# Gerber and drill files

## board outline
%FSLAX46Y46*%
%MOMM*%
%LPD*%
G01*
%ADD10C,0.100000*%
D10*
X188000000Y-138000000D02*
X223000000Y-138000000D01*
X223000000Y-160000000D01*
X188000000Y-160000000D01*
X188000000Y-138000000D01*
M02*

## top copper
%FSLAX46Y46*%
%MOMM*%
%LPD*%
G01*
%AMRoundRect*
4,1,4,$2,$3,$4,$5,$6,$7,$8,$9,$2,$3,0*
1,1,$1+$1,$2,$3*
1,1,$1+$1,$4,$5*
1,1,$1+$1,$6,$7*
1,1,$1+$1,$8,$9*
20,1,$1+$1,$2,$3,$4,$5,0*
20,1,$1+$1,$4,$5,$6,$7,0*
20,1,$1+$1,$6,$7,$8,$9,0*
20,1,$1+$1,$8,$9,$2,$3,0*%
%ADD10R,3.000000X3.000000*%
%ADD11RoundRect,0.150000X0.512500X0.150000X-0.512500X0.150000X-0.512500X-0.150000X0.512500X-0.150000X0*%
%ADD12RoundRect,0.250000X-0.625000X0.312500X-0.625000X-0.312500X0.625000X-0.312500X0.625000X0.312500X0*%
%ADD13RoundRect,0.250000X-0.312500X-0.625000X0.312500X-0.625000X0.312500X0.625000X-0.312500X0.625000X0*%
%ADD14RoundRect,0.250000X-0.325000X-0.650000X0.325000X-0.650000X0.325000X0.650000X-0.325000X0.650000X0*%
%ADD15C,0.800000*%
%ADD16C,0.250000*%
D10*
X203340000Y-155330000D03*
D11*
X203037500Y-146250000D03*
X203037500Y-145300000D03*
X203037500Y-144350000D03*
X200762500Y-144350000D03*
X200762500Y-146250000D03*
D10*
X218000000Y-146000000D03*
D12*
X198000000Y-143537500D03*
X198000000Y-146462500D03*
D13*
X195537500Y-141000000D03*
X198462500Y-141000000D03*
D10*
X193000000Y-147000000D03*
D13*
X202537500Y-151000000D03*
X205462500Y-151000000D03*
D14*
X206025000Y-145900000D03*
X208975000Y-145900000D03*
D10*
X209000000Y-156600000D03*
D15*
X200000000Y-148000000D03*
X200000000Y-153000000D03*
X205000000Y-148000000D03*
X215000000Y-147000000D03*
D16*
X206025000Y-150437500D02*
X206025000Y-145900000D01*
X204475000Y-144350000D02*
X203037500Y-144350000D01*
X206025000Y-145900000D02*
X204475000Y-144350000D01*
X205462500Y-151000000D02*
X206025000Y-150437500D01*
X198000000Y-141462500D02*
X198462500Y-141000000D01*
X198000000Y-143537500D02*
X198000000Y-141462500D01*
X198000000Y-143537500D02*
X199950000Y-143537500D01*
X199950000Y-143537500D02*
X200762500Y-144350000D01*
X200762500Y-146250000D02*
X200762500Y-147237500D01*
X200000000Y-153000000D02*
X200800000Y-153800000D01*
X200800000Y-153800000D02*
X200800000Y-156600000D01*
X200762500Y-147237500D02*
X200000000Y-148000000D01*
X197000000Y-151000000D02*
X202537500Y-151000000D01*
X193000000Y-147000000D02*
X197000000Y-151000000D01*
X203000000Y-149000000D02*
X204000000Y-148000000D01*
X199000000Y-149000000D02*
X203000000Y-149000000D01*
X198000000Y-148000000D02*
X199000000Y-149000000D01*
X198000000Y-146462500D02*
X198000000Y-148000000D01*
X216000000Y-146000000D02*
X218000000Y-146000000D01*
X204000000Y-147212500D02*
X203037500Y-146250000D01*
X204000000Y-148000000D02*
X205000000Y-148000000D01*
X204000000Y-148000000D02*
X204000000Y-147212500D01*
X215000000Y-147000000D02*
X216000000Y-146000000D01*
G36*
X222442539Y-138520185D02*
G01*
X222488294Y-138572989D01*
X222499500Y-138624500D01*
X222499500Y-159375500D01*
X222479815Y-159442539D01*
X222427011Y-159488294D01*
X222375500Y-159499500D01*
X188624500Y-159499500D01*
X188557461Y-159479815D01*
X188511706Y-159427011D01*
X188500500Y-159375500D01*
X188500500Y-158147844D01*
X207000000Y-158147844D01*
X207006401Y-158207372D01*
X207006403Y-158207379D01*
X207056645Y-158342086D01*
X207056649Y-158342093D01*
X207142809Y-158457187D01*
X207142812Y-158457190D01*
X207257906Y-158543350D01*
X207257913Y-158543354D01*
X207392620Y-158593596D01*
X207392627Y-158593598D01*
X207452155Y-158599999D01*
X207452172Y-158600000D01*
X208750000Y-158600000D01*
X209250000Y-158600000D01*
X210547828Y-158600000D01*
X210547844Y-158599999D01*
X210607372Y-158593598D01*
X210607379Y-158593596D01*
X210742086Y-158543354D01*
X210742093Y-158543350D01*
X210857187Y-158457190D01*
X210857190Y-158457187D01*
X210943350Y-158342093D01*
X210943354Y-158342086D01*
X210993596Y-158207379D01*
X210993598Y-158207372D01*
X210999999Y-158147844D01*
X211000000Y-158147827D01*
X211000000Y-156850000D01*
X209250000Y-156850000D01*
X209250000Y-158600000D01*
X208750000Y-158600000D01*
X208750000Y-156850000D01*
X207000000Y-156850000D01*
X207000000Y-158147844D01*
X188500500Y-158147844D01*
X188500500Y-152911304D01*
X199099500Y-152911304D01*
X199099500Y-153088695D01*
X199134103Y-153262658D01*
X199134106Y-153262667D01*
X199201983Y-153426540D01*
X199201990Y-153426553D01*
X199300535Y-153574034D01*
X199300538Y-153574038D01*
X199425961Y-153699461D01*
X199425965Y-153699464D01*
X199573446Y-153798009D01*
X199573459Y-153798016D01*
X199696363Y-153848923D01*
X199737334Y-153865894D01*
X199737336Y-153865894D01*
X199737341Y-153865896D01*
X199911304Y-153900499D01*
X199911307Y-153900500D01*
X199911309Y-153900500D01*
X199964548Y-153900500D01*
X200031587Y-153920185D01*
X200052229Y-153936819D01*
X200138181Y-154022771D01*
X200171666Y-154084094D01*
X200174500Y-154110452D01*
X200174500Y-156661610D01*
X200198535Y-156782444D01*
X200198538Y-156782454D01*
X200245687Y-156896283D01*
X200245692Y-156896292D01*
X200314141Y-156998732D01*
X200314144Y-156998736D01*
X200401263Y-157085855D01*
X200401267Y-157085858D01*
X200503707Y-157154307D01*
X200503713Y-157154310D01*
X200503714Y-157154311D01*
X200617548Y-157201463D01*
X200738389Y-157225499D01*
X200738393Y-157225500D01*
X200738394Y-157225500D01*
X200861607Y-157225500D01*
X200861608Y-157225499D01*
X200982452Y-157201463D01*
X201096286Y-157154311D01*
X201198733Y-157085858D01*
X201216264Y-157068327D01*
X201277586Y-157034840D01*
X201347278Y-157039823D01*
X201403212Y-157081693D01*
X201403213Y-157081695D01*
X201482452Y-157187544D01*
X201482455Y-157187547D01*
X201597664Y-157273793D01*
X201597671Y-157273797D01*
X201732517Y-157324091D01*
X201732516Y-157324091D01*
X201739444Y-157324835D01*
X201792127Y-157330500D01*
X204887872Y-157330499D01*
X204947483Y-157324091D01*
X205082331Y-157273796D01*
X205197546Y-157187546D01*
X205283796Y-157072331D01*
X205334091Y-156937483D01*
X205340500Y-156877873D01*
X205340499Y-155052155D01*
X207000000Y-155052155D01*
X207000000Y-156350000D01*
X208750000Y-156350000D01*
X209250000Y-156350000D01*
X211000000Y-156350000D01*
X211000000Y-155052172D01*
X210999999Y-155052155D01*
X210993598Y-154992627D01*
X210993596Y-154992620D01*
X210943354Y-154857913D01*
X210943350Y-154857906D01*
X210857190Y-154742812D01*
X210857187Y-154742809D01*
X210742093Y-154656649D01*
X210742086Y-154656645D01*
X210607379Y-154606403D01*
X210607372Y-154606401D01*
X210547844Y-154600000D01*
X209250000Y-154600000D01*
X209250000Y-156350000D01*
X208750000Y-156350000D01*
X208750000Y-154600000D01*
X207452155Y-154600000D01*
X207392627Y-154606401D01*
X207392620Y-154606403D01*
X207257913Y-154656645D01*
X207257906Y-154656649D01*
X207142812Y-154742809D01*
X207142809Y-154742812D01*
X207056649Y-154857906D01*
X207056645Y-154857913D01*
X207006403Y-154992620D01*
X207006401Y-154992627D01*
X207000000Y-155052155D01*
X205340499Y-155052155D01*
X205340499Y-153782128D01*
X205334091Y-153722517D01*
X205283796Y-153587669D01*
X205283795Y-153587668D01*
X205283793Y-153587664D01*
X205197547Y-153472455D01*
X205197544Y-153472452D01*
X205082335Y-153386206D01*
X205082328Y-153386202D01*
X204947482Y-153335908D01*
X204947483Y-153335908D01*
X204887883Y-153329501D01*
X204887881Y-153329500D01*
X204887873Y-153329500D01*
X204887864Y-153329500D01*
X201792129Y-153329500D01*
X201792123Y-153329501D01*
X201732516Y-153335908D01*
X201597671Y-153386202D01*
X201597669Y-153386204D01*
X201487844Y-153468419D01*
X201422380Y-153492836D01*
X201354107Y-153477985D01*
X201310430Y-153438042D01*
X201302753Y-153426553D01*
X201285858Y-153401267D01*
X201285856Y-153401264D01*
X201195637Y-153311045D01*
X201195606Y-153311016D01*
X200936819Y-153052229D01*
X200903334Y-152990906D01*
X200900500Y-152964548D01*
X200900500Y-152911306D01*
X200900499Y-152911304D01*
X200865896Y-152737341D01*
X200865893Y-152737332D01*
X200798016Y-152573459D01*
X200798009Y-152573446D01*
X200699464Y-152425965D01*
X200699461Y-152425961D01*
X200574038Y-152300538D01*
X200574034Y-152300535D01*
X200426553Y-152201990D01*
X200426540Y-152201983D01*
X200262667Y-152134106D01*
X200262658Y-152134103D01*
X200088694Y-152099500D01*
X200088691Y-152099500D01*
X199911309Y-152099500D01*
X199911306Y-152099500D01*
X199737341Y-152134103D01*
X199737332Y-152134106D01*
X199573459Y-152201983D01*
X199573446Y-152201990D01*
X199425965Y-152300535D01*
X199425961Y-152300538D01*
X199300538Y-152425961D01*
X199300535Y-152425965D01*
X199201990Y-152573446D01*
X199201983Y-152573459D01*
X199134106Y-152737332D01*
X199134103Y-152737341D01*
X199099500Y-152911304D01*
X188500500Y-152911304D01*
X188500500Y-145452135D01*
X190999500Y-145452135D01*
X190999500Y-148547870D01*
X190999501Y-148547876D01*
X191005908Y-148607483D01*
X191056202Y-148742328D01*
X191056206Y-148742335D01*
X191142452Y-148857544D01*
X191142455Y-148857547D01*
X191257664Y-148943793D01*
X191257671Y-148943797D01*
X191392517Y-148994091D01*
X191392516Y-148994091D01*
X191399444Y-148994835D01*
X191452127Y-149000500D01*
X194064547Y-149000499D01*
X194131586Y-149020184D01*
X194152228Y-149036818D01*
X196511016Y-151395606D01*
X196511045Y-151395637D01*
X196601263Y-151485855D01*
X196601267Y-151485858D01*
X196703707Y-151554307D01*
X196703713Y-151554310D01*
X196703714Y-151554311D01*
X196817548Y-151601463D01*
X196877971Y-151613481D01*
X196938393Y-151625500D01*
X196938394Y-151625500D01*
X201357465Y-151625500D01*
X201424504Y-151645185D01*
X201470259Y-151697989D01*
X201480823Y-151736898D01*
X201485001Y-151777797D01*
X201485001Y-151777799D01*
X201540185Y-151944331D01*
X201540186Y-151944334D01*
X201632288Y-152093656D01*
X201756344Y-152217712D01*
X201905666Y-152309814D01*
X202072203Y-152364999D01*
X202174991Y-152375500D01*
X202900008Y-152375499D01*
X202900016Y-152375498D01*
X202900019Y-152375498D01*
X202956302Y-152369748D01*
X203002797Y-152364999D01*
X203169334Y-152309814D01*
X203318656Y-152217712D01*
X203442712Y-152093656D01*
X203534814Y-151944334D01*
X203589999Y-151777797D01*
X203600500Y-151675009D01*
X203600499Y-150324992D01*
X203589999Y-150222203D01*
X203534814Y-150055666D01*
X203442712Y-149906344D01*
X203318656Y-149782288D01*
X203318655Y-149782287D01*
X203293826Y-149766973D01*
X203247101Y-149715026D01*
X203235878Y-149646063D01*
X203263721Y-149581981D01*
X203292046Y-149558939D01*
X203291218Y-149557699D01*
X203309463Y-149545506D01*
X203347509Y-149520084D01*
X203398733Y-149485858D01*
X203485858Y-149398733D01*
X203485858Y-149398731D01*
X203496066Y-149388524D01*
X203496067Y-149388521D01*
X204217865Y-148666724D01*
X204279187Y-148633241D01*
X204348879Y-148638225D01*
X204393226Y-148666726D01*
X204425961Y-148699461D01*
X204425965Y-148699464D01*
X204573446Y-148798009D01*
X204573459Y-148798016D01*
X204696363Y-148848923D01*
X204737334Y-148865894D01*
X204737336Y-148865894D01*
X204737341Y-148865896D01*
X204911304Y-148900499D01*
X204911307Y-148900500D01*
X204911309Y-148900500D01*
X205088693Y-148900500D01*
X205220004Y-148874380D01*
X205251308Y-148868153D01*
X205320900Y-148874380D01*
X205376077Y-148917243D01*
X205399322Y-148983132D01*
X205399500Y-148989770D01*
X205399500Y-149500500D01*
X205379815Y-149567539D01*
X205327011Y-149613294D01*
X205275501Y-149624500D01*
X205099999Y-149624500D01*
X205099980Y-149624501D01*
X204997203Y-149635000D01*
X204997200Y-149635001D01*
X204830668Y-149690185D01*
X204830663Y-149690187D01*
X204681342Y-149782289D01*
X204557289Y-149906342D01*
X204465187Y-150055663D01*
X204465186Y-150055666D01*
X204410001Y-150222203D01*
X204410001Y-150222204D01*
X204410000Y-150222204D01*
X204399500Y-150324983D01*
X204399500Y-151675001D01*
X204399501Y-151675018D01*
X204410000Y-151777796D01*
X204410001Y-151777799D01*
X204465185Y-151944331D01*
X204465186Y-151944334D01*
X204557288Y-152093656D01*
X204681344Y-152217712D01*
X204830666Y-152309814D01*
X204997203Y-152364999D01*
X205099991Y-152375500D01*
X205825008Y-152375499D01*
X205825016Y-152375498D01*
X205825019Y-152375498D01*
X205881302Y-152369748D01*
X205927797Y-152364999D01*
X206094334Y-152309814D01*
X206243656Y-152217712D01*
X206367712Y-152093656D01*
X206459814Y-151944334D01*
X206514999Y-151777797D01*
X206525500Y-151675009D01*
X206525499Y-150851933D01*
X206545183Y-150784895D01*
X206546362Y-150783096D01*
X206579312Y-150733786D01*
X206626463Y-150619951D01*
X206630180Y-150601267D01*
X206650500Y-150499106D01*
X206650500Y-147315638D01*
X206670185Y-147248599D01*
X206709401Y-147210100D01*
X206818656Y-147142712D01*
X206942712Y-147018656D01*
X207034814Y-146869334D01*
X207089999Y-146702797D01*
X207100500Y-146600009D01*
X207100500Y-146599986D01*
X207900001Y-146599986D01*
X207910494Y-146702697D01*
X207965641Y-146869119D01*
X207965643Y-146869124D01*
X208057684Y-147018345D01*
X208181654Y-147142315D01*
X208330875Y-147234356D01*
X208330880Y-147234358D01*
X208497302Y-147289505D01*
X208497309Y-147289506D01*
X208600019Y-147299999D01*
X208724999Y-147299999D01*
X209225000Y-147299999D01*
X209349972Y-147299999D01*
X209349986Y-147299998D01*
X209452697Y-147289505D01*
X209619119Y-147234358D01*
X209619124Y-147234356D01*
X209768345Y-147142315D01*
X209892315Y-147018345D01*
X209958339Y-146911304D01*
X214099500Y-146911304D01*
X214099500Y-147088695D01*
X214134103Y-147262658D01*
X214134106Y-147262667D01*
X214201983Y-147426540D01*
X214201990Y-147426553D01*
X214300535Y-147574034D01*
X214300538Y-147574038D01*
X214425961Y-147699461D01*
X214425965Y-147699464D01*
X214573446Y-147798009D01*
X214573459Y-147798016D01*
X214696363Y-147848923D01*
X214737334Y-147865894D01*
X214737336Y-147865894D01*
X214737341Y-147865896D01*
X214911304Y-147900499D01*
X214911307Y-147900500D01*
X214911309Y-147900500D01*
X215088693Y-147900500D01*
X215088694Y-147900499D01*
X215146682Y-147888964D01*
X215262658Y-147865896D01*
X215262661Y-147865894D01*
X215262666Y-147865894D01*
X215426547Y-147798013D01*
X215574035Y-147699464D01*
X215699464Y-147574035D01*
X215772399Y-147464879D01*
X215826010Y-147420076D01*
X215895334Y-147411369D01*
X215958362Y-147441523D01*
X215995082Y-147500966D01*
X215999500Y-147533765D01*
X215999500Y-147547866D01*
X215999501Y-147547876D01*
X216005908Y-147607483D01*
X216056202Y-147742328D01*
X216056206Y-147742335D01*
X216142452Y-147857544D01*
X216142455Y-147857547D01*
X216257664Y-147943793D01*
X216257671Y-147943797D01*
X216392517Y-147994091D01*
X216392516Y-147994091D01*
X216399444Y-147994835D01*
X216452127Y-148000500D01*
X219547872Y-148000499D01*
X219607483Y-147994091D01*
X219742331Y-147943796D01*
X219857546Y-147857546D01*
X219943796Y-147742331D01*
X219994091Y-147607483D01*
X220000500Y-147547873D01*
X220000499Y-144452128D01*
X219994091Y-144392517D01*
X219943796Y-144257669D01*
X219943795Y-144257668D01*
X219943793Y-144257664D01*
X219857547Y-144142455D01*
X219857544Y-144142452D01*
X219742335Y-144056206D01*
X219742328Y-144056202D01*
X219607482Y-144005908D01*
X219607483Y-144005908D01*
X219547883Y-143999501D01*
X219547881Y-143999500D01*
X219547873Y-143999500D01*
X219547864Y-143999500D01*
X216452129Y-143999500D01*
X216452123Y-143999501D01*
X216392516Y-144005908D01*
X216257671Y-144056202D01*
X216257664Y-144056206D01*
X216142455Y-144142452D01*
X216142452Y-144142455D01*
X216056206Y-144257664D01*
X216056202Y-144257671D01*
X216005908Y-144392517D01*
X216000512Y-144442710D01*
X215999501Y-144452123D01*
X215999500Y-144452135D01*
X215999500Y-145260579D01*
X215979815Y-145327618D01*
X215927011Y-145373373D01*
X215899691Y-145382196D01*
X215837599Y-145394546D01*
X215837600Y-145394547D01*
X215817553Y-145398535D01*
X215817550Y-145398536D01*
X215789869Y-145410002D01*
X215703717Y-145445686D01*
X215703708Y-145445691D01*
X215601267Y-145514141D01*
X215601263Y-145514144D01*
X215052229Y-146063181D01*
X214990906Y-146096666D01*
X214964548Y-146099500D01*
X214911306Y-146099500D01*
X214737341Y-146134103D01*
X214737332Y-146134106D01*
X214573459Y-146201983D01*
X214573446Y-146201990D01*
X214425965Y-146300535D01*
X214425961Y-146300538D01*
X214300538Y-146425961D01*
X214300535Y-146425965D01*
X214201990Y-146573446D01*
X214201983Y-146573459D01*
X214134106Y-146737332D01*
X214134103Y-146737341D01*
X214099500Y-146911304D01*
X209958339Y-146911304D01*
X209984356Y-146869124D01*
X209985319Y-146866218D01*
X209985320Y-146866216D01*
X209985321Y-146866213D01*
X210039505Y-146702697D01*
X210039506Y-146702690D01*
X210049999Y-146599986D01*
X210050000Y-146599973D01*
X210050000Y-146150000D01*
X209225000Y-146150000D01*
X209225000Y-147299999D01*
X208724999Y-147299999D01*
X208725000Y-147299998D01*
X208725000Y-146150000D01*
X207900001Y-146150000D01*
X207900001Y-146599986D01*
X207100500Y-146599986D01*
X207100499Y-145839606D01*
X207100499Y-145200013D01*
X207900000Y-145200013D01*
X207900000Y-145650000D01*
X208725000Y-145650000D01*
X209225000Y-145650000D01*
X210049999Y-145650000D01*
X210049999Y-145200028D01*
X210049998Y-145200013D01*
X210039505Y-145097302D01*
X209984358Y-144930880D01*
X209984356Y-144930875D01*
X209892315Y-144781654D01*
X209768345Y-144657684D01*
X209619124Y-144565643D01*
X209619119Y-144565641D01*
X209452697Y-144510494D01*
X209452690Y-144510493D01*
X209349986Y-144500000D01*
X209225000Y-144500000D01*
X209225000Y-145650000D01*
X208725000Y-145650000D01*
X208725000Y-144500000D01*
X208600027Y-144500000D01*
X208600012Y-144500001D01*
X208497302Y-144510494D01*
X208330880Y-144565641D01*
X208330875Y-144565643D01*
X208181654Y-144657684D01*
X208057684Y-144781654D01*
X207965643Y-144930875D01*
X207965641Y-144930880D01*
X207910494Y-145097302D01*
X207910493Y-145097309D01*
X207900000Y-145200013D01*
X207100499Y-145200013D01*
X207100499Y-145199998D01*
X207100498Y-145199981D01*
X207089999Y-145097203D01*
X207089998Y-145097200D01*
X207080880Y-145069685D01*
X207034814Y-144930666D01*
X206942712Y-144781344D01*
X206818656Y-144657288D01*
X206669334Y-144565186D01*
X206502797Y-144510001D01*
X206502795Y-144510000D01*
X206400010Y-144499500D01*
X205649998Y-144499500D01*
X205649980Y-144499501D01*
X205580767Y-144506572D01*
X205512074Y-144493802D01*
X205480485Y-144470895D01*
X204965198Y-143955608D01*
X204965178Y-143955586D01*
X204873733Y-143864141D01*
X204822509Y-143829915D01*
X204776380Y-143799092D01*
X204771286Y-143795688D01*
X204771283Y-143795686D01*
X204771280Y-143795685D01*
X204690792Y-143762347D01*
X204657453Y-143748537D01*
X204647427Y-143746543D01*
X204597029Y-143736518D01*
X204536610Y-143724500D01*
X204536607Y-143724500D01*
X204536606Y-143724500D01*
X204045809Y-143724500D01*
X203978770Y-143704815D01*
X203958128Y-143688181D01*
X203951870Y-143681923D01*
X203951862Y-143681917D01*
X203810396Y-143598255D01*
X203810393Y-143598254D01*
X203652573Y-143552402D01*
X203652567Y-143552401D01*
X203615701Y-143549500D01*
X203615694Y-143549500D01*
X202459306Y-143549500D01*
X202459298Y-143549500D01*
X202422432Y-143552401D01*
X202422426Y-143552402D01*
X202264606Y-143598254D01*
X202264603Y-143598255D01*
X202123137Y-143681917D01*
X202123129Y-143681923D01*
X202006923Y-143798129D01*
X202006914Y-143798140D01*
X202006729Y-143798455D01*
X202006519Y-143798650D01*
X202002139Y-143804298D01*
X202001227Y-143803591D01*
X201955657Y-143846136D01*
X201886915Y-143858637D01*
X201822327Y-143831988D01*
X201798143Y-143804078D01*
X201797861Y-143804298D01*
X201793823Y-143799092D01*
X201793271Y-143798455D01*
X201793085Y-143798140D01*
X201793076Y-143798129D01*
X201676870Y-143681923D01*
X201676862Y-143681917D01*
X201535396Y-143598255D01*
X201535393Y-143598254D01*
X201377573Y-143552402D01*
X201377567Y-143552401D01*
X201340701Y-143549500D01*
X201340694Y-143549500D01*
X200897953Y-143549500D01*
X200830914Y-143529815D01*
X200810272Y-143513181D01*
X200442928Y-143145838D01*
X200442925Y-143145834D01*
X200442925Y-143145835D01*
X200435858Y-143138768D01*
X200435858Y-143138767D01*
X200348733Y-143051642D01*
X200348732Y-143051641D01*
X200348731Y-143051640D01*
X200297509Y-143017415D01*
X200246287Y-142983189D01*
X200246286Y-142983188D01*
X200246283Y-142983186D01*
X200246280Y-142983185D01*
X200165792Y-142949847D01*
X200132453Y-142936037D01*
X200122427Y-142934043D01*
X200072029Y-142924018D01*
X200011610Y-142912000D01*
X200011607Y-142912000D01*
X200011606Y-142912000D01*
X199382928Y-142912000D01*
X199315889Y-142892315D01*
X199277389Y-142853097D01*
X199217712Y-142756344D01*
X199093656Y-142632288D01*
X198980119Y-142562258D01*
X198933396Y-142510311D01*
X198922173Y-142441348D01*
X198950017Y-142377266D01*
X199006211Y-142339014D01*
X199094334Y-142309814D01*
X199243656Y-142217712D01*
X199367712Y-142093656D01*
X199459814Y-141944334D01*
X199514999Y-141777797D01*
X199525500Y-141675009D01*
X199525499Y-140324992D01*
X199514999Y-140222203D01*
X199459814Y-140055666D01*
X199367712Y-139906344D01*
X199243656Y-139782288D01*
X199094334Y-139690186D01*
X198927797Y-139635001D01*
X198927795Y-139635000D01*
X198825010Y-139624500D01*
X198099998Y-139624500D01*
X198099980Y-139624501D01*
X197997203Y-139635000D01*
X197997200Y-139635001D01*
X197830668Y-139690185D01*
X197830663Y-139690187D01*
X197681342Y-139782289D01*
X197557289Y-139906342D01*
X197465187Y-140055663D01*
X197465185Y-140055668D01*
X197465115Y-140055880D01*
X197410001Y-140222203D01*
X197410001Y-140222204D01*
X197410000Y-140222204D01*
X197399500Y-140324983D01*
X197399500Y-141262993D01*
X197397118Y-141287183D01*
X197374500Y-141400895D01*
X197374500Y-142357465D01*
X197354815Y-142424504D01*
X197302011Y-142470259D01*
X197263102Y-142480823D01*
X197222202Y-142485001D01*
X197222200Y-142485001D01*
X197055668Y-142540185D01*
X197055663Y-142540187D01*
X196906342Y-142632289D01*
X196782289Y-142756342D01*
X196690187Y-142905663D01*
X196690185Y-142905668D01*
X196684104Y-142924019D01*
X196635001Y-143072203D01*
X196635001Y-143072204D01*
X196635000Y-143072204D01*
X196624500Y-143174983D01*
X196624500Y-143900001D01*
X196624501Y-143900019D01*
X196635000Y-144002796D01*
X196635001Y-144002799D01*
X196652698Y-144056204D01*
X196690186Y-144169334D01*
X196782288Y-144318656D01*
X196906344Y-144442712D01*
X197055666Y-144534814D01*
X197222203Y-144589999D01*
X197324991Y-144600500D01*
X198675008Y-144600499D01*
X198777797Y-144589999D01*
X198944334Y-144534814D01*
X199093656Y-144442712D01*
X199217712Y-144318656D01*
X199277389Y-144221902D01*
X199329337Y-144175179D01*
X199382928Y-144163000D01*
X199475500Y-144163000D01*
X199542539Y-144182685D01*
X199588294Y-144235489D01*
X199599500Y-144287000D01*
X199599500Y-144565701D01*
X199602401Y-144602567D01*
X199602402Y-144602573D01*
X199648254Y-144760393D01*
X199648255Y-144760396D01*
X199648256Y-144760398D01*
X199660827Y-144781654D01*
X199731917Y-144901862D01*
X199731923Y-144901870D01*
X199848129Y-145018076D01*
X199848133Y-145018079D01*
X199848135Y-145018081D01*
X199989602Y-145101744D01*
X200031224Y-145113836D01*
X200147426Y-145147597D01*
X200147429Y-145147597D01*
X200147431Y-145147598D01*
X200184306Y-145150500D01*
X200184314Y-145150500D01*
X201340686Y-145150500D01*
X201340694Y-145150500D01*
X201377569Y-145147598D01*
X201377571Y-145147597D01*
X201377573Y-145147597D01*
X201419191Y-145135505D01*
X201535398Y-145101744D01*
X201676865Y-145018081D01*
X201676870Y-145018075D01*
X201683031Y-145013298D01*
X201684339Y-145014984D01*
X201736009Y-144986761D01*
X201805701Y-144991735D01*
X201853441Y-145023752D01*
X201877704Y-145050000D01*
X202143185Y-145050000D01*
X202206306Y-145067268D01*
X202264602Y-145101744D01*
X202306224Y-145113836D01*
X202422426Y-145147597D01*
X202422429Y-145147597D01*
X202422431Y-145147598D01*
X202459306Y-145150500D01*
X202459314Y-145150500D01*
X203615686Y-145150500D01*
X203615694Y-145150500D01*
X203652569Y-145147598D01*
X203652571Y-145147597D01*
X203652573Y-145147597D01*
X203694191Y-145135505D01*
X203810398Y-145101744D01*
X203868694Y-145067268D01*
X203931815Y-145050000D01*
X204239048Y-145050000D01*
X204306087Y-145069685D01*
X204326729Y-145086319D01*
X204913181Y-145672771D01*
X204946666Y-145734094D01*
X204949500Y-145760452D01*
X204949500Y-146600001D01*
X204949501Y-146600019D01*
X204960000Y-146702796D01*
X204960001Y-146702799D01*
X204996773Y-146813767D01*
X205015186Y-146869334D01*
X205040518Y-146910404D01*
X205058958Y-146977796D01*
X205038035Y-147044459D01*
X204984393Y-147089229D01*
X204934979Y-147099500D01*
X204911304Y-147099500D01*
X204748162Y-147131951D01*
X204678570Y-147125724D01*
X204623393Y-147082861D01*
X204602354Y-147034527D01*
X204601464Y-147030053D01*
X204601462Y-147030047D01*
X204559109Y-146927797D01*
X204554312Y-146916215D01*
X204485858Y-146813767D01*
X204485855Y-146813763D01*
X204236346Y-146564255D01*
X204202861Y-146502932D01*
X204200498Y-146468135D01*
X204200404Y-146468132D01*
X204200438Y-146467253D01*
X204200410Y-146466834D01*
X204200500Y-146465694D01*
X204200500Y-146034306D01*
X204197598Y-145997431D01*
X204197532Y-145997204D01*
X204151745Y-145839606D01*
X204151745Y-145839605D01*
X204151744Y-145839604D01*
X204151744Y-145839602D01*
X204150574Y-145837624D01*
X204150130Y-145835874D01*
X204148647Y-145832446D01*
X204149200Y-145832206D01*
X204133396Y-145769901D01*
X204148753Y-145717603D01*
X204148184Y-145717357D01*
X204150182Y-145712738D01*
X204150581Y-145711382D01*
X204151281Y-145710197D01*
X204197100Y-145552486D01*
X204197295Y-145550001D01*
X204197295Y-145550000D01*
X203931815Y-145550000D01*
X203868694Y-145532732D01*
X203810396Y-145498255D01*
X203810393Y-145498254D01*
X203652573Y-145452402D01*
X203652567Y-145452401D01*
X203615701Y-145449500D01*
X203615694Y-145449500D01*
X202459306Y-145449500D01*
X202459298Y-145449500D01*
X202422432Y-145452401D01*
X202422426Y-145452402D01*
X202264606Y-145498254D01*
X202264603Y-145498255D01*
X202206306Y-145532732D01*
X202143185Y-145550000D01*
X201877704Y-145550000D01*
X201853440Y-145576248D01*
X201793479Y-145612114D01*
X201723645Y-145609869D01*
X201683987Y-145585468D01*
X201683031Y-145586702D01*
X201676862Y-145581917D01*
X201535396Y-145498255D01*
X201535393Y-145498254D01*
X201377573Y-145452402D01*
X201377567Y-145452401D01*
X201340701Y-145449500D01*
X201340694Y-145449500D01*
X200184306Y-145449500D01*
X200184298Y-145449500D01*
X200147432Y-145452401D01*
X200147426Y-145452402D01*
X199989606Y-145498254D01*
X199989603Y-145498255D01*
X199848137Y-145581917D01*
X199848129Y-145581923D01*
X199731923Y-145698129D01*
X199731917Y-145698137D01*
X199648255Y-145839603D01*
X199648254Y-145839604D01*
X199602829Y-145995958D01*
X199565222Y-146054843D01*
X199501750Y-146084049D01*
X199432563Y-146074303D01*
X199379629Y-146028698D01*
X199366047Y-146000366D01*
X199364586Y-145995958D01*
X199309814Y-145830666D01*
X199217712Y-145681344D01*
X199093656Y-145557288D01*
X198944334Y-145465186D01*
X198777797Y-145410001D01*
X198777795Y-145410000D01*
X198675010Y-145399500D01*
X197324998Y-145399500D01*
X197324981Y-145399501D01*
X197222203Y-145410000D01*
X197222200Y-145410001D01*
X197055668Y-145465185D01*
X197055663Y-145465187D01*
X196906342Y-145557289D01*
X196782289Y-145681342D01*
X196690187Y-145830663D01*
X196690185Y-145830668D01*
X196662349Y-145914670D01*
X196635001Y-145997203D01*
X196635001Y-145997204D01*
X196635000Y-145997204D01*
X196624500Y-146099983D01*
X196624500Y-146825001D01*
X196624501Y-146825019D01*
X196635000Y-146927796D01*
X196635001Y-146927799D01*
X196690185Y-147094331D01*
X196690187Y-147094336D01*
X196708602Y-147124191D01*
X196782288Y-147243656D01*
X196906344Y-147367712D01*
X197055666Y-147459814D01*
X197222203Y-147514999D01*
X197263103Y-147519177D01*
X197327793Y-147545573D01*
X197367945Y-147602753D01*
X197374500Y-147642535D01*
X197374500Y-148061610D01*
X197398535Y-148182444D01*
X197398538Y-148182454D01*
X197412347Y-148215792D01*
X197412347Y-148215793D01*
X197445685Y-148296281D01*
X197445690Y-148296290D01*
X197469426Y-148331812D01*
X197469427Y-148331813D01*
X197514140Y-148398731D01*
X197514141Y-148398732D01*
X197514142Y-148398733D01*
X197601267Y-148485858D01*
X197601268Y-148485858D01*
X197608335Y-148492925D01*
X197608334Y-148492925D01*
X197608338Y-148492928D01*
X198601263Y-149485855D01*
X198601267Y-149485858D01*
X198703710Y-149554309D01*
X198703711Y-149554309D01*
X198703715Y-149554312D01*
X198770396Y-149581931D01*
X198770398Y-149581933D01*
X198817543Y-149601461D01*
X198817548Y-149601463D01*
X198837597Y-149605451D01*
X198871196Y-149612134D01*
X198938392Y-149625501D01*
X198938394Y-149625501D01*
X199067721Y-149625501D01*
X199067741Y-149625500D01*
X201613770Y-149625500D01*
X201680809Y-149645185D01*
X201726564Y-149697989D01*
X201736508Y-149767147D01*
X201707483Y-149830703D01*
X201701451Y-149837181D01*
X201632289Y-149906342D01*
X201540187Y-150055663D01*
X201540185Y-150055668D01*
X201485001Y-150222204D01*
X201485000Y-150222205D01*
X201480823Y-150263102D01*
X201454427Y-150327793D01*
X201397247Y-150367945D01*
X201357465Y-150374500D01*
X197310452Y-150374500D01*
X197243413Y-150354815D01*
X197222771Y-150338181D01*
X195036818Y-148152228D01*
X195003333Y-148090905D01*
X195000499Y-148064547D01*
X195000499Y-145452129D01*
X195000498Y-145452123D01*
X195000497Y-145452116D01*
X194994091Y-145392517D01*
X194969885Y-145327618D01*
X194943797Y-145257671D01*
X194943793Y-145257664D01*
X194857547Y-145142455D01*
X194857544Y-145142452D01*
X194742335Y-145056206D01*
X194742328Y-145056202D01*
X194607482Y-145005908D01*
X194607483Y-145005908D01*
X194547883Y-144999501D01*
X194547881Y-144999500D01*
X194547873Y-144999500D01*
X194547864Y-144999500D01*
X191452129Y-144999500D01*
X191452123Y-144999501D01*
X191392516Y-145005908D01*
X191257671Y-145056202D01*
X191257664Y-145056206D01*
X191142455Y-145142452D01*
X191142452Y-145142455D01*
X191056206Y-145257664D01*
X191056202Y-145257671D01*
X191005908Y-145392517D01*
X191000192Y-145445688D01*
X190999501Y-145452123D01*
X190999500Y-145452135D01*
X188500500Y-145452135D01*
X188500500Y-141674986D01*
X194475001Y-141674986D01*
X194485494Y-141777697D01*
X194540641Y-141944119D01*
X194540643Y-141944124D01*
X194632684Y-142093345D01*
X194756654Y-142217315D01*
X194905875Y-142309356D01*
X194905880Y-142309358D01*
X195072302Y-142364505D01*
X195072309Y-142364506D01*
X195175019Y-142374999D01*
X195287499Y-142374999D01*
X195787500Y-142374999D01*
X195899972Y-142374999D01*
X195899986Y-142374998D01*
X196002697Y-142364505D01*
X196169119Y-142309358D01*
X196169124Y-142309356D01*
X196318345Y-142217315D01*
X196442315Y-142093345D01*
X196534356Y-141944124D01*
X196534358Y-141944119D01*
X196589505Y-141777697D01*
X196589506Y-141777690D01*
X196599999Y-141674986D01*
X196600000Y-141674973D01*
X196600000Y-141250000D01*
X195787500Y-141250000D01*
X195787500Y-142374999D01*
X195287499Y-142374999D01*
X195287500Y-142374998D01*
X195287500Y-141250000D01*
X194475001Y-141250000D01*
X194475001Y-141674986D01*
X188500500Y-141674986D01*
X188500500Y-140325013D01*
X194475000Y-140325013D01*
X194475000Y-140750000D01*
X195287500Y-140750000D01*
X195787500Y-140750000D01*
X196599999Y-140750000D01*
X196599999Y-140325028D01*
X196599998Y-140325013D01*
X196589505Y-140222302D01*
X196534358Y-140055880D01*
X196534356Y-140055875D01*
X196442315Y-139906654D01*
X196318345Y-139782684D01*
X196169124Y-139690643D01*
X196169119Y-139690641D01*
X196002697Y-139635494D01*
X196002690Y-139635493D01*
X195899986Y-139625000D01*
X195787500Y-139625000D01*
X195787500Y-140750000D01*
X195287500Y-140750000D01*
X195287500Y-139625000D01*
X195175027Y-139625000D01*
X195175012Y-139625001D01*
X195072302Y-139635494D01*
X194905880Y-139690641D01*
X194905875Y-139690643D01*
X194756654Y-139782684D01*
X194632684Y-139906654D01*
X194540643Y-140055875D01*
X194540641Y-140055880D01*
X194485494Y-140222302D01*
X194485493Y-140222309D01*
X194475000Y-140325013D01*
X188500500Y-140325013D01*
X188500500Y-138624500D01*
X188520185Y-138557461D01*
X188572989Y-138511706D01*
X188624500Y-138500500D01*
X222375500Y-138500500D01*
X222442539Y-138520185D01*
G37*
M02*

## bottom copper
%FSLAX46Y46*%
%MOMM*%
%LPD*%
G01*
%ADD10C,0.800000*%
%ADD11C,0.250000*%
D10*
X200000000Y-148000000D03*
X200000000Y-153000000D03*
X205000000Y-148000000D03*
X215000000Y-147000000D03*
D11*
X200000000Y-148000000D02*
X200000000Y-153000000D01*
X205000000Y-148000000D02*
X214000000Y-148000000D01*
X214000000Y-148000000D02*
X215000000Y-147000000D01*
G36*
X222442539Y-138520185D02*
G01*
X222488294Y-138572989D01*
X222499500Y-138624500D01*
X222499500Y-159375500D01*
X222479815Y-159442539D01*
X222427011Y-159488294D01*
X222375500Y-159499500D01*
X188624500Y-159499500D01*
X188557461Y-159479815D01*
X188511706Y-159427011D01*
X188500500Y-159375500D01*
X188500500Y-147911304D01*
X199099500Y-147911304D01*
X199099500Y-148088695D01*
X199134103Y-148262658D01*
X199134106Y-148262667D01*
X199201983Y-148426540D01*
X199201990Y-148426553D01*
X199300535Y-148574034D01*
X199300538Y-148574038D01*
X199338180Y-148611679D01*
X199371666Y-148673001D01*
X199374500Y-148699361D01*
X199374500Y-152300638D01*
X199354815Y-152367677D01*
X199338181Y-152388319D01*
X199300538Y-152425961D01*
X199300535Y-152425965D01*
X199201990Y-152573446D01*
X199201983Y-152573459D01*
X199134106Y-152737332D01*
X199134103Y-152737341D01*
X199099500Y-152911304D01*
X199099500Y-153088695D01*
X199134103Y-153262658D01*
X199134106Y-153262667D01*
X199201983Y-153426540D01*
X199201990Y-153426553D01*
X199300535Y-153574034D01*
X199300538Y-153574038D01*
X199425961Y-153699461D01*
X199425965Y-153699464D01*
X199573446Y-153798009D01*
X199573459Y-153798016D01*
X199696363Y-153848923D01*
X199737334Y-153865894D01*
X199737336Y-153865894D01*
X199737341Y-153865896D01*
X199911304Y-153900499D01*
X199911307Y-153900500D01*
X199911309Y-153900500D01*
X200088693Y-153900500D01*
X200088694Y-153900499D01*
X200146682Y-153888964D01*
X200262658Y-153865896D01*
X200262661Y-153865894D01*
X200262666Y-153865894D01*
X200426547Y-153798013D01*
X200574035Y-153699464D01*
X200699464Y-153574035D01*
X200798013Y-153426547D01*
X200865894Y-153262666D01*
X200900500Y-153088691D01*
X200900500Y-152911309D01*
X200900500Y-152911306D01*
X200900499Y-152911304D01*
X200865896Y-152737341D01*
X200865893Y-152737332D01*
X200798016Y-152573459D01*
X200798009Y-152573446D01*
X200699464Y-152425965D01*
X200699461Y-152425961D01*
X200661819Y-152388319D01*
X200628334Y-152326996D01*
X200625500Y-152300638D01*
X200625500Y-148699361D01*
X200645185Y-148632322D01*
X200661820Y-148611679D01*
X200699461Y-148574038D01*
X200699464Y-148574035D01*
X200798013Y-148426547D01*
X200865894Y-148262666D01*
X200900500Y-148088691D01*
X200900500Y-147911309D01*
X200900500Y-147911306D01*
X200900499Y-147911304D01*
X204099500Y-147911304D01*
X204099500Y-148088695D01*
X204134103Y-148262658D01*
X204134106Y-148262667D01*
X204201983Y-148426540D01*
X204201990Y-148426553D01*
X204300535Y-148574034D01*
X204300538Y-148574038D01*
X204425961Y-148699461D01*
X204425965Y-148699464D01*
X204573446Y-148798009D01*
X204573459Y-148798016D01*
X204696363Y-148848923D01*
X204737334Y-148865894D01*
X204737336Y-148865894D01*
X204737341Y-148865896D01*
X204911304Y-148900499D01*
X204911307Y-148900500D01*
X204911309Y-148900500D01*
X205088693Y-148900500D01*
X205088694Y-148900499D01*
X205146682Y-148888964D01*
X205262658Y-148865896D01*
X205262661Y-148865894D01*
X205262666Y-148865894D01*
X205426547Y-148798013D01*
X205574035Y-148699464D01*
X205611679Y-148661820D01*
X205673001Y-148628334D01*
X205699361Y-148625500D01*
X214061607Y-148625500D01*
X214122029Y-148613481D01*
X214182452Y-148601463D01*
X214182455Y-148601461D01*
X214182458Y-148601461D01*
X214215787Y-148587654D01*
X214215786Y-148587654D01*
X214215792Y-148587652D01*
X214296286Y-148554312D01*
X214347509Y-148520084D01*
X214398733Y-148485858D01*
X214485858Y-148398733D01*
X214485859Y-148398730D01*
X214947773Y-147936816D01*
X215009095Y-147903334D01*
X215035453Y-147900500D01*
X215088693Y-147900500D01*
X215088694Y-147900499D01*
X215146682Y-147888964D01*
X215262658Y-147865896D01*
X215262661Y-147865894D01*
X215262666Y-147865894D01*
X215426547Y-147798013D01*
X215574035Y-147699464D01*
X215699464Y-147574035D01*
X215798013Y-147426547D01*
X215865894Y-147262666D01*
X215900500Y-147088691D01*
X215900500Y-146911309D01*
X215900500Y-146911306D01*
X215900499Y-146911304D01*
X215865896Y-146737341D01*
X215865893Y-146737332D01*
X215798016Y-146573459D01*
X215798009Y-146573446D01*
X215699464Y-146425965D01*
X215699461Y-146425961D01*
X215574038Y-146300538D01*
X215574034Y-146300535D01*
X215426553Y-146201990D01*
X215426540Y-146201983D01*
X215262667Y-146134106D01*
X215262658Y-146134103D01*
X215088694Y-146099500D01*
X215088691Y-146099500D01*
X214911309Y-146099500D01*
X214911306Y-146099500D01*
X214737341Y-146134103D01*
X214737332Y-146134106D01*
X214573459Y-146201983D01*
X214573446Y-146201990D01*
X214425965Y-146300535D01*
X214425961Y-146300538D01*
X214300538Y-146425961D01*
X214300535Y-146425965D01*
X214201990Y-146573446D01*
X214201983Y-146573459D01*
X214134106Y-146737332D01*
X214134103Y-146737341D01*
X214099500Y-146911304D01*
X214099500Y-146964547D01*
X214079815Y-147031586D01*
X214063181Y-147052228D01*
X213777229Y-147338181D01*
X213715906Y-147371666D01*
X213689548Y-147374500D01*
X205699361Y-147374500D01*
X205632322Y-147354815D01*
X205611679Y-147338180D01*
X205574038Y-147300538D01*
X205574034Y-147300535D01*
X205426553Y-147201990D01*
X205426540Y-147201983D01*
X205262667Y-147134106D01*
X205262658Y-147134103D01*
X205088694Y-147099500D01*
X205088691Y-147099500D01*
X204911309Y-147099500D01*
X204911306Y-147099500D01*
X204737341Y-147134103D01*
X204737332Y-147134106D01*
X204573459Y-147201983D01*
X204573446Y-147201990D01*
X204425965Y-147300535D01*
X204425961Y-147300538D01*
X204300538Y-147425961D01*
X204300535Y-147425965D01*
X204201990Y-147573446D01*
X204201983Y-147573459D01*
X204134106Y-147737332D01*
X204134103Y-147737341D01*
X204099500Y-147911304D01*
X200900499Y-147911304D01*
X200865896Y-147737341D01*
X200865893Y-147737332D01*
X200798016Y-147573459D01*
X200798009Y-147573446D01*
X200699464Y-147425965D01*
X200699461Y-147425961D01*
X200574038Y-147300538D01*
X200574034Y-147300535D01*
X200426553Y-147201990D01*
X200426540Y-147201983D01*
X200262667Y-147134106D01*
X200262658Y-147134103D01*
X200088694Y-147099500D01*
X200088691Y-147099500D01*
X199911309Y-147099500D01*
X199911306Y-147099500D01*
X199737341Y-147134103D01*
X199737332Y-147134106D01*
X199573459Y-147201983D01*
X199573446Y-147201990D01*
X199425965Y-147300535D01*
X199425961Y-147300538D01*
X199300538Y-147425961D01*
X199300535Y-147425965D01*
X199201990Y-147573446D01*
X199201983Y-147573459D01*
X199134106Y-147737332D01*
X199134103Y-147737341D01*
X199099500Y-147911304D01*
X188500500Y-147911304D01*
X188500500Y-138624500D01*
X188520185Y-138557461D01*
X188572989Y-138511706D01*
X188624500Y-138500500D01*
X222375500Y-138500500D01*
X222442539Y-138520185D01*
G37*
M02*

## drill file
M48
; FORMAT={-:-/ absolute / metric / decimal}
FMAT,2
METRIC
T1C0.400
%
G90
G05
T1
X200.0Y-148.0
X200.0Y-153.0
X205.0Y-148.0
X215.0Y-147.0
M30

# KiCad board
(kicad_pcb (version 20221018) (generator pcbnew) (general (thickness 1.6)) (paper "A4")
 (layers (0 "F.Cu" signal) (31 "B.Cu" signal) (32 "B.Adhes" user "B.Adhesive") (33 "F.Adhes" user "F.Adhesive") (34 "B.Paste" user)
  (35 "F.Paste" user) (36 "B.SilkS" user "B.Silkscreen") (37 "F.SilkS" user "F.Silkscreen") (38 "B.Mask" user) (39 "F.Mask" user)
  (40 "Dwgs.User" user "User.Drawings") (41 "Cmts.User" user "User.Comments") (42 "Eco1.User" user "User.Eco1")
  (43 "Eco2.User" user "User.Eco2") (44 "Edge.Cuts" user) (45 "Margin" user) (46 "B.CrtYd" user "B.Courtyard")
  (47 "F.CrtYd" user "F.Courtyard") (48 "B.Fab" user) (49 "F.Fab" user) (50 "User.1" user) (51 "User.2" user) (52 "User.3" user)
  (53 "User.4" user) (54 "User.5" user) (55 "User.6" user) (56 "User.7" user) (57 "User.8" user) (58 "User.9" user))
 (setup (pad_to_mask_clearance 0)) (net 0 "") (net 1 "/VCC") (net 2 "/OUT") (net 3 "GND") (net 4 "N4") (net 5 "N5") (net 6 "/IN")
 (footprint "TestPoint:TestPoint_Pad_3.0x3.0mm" (layer "F.Cu") (at 203.34 155.33)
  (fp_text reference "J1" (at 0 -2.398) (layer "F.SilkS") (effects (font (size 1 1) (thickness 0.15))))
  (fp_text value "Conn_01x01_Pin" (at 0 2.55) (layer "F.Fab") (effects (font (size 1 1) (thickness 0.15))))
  (pad "1" smd rect (at 0 0) (size 3 3) (layers "F.Cu" "F.Mask") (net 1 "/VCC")))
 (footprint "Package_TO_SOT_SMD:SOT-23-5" (layer "F.Cu") (at 201.9 145.3 180)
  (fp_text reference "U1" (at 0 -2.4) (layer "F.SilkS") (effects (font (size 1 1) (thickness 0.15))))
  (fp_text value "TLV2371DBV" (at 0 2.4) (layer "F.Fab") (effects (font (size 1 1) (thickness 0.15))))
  (pad "1" smd roundrect (at -1.1375 -0.95 180) (size 1.325 0.6) (layers "F.Cu" "F.Paste" "F.Mask") (roundrect_rratio 0.25) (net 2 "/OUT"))
  (pad "2" smd roundrect (at -1.1375 0 180) (size 1.325 0.6) (layers "F.Cu" "F.Paste" "F.Mask") (roundrect_rratio 0.25) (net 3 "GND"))
  (pad "3" smd roundrect (at -1.1375 0.95 180) (size 1.325 0.6) (layers "F.Cu" "F.Paste" "F.Mask") (roundrect_rratio 0.25) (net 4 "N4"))
  (pad "4" smd roundrect (at 1.1375 0.95 180) (size 1.325 0.6) (layers "F.Cu" "F.Paste" "F.Mask") (roundrect_rratio 0.25) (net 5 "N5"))
  (pad "5" smd roundrect (at 1.1375 -0.95 180) (size 1.325 0.6) (layers "F.Cu" "F.Paste" "F.Mask") (roundrect_rratio 0.25) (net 1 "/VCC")))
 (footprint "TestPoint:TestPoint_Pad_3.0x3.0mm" (layer "F.Cu") (at 218 146)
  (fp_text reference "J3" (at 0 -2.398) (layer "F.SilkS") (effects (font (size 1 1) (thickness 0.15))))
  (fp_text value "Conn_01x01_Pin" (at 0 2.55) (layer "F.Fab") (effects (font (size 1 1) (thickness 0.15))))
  (pad "1" smd rect (at 0 0) (size 3 3) (layers "F.Cu" "F.Mask") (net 2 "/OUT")))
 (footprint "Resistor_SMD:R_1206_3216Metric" (layer "F.Cu") (at 198 145 -90)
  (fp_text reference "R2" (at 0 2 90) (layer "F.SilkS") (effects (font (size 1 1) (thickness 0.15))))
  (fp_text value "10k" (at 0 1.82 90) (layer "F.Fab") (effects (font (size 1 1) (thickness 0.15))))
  (pad "1" smd roundrect (at -1.4625 0 270) (size 1.125 1.75) (layers "F.Cu" "F.Paste" "F.Mask") (roundrect_rratio 0.222222) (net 5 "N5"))
  (pad "2" smd roundrect (at 1.4625 0 270) (size 1.125 1.75) (layers "F.Cu" "F.Paste" "F.Mask") (roundrect_rratio 0.222222) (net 2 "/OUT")))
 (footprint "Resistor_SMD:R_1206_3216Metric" (layer "F.Cu") (at 197 141)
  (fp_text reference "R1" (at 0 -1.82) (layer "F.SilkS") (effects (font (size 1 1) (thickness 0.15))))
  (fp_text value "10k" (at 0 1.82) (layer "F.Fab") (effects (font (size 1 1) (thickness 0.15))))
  (pad "1" smd roundrect (at -1.4625 0) (size 1.125 1.75) (layers "F.Cu" "F.Paste" "F.Mask") (roundrect_rratio 0.222222) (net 3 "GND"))
  (pad "2" smd roundrect (at 1.4625 0) (size 1.125 1.75) (layers "F.Cu" "F.Paste" "F.Mask") (roundrect_rratio 0.222222) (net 5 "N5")))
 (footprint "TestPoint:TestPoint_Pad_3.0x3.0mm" (layer "F.Cu") (at 193 147)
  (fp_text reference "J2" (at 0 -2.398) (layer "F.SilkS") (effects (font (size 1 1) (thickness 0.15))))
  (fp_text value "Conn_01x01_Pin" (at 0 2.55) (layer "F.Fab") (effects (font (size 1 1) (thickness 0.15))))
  (pad "1" smd rect (at 0 0) (size 3 3) (layers "F.Cu" "F.Mask") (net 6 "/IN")))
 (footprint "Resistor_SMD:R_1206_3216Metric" (layer "F.Cu") (at 204 151)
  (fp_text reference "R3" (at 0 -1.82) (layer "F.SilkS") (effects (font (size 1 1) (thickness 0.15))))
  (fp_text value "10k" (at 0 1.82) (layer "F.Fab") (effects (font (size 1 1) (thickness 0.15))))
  (pad "1" smd roundrect (at -1.4625 0) (size 1.125 1.75) (layers "F.Cu" "F.Paste" "F.Mask") (roundrect_rratio 0.222222) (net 6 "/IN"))
  (pad "2" smd roundrect (at 1.4625 0) (size 1.125 1.75) (layers "F.Cu" "F.Paste" "F.Mask") (roundrect_rratio 0.222222) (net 4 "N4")))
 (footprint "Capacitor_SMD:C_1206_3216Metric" (layer "F.Cu") (at 207.5 145.9)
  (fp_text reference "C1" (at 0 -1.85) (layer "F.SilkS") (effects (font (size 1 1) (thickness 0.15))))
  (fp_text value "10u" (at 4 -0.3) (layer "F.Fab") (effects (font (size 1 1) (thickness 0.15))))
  (pad "1" smd roundrect (at -1.475 0) (size 1.15 1.8) (layers "F.Cu" "F.Paste" "F.Mask") (roundrect_rratio 0.217391) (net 4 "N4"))
  (pad "2" smd roundrect (at 1.475 0) (size 1.15 1.8) (layers "F.Cu" "F.Paste" "F.Mask") (roundrect_rratio 0.217391) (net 3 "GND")))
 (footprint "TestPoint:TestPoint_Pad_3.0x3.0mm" (layer "F.Cu") (at 209 156.6)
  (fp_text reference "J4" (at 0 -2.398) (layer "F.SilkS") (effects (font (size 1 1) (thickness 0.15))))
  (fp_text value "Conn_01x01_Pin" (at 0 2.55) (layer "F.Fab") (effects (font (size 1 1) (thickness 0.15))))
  (pad "1" smd rect (at 0 0) (size 3 3) (layers "F.Cu" "F.Mask") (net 3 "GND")))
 (gr_rect (start 188 138) (end 223 160) (stroke (width 0.1) (type default)) (fill none) (layer "Edge.Cuts"))
 (segment (start 206.025 150.4375) (end 206.025 145.9) (width 0.25) (layer "F.Cu") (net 4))
 (segment (start 204.475 144.35) (end 203.0375 144.35) (width 0.25) (layer "F.Cu") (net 4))
 (segment (start 206.025 145.9) (end 204.475 144.35) (width 0.25) (layer "F.Cu") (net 4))
 (segment (start 205.4625 151) (end 206.025 150.4375) (width 0.25) (layer "F.Cu") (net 4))
 (segment (start 198 141.4625) (end 198.4625 141) (width 0.25) (layer "F.Cu") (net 5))
 (segment (start 198 143.5375) (end 198 141.4625) (width 0.25) (layer "F.Cu") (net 5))
 (segment (start 198 143.5375) (end 199.95 143.5375) (width 0.25) (layer "F.Cu") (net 5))
 (segment (start 199.95 143.5375) (end 200.7625 144.35) (width 0.25) (layer "F.Cu") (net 5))
 (segment (start 200.7625 146.25) (end 200.7625 147.2375) (width 0.25) (layer "F.Cu") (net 1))
 (segment (start 200 153) (end 200.8 153.8) (width 0.25) (layer "F.Cu") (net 1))
 (segment (start 200.8 153.8) (end 200.8 156.6) (width 0.25) (layer "F.Cu") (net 1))
 (segment (start 200.7625 147.2375) (end 200 148) (width 0.25) (layer "F.Cu") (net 1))
 (via (at 200 148) (size 0.8) (drill 0.4) (layers "F.Cu" "B.Cu") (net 1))
 (via (at 200 153) (size 0.8) (drill 0.4) (layers "F.Cu" "B.Cu") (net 1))
 (segment (start 200 148) (end 200 153) (width 0.25) (layer "B.Cu") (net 1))
 (segment (start 197 151) (end 202.5375 151) (width 0.25) (layer "F.Cu") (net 6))
 (segment (start 193 147) (end 197 151) (width 0.25) (layer "F.Cu") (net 6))
 (segment (start 203 149) (end 204 148) (width 0.25) (layer "F.Cu") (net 2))
 (segment (start 199 149) (end 203 149) (width 0.25) (layer "F.Cu") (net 2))
 (segment (start 198 148) (end 199 149) (width 0.25) (layer "F.Cu") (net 2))
 (segment (start 198 146.4625) (end 198 148) (width 0.25) (layer "F.Cu") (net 2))
 (segment (start 216 146) (end 218 146) (width 0.25) (layer "F.Cu") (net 2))
 (segment (start 204 147.2125) (end 203.0375 146.25) (width 0.25) (layer "F.Cu") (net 2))
 (segment (start 204 148) (end 205 148) (width 0.25) (layer "F.Cu") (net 2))
 (segment (start 204 148) (end 204 147.2125) (width 0.25) (layer "F.Cu") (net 2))
 (segment (start 215 147) (end 216 146) (width 0.25) (layer "F.Cu") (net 2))
 (via (at 205 148) (size 0.8) (drill 0.4) (layers "F.Cu" "B.Cu") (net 2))
 (via (at 215 147) (size 0.8) (drill 0.4) (layers "F.Cu" "B.Cu") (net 2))
 (segment (start 205 148) (end 214 148) (width 0.25) (layer "B.Cu") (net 2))
 (segment (start 214 148) (end 215 147) (width 0.25) (layer "B.Cu") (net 2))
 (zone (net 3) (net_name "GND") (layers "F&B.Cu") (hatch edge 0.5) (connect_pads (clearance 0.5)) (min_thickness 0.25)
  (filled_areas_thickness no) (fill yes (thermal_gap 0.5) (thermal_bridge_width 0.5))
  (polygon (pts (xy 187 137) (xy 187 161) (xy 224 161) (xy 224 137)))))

